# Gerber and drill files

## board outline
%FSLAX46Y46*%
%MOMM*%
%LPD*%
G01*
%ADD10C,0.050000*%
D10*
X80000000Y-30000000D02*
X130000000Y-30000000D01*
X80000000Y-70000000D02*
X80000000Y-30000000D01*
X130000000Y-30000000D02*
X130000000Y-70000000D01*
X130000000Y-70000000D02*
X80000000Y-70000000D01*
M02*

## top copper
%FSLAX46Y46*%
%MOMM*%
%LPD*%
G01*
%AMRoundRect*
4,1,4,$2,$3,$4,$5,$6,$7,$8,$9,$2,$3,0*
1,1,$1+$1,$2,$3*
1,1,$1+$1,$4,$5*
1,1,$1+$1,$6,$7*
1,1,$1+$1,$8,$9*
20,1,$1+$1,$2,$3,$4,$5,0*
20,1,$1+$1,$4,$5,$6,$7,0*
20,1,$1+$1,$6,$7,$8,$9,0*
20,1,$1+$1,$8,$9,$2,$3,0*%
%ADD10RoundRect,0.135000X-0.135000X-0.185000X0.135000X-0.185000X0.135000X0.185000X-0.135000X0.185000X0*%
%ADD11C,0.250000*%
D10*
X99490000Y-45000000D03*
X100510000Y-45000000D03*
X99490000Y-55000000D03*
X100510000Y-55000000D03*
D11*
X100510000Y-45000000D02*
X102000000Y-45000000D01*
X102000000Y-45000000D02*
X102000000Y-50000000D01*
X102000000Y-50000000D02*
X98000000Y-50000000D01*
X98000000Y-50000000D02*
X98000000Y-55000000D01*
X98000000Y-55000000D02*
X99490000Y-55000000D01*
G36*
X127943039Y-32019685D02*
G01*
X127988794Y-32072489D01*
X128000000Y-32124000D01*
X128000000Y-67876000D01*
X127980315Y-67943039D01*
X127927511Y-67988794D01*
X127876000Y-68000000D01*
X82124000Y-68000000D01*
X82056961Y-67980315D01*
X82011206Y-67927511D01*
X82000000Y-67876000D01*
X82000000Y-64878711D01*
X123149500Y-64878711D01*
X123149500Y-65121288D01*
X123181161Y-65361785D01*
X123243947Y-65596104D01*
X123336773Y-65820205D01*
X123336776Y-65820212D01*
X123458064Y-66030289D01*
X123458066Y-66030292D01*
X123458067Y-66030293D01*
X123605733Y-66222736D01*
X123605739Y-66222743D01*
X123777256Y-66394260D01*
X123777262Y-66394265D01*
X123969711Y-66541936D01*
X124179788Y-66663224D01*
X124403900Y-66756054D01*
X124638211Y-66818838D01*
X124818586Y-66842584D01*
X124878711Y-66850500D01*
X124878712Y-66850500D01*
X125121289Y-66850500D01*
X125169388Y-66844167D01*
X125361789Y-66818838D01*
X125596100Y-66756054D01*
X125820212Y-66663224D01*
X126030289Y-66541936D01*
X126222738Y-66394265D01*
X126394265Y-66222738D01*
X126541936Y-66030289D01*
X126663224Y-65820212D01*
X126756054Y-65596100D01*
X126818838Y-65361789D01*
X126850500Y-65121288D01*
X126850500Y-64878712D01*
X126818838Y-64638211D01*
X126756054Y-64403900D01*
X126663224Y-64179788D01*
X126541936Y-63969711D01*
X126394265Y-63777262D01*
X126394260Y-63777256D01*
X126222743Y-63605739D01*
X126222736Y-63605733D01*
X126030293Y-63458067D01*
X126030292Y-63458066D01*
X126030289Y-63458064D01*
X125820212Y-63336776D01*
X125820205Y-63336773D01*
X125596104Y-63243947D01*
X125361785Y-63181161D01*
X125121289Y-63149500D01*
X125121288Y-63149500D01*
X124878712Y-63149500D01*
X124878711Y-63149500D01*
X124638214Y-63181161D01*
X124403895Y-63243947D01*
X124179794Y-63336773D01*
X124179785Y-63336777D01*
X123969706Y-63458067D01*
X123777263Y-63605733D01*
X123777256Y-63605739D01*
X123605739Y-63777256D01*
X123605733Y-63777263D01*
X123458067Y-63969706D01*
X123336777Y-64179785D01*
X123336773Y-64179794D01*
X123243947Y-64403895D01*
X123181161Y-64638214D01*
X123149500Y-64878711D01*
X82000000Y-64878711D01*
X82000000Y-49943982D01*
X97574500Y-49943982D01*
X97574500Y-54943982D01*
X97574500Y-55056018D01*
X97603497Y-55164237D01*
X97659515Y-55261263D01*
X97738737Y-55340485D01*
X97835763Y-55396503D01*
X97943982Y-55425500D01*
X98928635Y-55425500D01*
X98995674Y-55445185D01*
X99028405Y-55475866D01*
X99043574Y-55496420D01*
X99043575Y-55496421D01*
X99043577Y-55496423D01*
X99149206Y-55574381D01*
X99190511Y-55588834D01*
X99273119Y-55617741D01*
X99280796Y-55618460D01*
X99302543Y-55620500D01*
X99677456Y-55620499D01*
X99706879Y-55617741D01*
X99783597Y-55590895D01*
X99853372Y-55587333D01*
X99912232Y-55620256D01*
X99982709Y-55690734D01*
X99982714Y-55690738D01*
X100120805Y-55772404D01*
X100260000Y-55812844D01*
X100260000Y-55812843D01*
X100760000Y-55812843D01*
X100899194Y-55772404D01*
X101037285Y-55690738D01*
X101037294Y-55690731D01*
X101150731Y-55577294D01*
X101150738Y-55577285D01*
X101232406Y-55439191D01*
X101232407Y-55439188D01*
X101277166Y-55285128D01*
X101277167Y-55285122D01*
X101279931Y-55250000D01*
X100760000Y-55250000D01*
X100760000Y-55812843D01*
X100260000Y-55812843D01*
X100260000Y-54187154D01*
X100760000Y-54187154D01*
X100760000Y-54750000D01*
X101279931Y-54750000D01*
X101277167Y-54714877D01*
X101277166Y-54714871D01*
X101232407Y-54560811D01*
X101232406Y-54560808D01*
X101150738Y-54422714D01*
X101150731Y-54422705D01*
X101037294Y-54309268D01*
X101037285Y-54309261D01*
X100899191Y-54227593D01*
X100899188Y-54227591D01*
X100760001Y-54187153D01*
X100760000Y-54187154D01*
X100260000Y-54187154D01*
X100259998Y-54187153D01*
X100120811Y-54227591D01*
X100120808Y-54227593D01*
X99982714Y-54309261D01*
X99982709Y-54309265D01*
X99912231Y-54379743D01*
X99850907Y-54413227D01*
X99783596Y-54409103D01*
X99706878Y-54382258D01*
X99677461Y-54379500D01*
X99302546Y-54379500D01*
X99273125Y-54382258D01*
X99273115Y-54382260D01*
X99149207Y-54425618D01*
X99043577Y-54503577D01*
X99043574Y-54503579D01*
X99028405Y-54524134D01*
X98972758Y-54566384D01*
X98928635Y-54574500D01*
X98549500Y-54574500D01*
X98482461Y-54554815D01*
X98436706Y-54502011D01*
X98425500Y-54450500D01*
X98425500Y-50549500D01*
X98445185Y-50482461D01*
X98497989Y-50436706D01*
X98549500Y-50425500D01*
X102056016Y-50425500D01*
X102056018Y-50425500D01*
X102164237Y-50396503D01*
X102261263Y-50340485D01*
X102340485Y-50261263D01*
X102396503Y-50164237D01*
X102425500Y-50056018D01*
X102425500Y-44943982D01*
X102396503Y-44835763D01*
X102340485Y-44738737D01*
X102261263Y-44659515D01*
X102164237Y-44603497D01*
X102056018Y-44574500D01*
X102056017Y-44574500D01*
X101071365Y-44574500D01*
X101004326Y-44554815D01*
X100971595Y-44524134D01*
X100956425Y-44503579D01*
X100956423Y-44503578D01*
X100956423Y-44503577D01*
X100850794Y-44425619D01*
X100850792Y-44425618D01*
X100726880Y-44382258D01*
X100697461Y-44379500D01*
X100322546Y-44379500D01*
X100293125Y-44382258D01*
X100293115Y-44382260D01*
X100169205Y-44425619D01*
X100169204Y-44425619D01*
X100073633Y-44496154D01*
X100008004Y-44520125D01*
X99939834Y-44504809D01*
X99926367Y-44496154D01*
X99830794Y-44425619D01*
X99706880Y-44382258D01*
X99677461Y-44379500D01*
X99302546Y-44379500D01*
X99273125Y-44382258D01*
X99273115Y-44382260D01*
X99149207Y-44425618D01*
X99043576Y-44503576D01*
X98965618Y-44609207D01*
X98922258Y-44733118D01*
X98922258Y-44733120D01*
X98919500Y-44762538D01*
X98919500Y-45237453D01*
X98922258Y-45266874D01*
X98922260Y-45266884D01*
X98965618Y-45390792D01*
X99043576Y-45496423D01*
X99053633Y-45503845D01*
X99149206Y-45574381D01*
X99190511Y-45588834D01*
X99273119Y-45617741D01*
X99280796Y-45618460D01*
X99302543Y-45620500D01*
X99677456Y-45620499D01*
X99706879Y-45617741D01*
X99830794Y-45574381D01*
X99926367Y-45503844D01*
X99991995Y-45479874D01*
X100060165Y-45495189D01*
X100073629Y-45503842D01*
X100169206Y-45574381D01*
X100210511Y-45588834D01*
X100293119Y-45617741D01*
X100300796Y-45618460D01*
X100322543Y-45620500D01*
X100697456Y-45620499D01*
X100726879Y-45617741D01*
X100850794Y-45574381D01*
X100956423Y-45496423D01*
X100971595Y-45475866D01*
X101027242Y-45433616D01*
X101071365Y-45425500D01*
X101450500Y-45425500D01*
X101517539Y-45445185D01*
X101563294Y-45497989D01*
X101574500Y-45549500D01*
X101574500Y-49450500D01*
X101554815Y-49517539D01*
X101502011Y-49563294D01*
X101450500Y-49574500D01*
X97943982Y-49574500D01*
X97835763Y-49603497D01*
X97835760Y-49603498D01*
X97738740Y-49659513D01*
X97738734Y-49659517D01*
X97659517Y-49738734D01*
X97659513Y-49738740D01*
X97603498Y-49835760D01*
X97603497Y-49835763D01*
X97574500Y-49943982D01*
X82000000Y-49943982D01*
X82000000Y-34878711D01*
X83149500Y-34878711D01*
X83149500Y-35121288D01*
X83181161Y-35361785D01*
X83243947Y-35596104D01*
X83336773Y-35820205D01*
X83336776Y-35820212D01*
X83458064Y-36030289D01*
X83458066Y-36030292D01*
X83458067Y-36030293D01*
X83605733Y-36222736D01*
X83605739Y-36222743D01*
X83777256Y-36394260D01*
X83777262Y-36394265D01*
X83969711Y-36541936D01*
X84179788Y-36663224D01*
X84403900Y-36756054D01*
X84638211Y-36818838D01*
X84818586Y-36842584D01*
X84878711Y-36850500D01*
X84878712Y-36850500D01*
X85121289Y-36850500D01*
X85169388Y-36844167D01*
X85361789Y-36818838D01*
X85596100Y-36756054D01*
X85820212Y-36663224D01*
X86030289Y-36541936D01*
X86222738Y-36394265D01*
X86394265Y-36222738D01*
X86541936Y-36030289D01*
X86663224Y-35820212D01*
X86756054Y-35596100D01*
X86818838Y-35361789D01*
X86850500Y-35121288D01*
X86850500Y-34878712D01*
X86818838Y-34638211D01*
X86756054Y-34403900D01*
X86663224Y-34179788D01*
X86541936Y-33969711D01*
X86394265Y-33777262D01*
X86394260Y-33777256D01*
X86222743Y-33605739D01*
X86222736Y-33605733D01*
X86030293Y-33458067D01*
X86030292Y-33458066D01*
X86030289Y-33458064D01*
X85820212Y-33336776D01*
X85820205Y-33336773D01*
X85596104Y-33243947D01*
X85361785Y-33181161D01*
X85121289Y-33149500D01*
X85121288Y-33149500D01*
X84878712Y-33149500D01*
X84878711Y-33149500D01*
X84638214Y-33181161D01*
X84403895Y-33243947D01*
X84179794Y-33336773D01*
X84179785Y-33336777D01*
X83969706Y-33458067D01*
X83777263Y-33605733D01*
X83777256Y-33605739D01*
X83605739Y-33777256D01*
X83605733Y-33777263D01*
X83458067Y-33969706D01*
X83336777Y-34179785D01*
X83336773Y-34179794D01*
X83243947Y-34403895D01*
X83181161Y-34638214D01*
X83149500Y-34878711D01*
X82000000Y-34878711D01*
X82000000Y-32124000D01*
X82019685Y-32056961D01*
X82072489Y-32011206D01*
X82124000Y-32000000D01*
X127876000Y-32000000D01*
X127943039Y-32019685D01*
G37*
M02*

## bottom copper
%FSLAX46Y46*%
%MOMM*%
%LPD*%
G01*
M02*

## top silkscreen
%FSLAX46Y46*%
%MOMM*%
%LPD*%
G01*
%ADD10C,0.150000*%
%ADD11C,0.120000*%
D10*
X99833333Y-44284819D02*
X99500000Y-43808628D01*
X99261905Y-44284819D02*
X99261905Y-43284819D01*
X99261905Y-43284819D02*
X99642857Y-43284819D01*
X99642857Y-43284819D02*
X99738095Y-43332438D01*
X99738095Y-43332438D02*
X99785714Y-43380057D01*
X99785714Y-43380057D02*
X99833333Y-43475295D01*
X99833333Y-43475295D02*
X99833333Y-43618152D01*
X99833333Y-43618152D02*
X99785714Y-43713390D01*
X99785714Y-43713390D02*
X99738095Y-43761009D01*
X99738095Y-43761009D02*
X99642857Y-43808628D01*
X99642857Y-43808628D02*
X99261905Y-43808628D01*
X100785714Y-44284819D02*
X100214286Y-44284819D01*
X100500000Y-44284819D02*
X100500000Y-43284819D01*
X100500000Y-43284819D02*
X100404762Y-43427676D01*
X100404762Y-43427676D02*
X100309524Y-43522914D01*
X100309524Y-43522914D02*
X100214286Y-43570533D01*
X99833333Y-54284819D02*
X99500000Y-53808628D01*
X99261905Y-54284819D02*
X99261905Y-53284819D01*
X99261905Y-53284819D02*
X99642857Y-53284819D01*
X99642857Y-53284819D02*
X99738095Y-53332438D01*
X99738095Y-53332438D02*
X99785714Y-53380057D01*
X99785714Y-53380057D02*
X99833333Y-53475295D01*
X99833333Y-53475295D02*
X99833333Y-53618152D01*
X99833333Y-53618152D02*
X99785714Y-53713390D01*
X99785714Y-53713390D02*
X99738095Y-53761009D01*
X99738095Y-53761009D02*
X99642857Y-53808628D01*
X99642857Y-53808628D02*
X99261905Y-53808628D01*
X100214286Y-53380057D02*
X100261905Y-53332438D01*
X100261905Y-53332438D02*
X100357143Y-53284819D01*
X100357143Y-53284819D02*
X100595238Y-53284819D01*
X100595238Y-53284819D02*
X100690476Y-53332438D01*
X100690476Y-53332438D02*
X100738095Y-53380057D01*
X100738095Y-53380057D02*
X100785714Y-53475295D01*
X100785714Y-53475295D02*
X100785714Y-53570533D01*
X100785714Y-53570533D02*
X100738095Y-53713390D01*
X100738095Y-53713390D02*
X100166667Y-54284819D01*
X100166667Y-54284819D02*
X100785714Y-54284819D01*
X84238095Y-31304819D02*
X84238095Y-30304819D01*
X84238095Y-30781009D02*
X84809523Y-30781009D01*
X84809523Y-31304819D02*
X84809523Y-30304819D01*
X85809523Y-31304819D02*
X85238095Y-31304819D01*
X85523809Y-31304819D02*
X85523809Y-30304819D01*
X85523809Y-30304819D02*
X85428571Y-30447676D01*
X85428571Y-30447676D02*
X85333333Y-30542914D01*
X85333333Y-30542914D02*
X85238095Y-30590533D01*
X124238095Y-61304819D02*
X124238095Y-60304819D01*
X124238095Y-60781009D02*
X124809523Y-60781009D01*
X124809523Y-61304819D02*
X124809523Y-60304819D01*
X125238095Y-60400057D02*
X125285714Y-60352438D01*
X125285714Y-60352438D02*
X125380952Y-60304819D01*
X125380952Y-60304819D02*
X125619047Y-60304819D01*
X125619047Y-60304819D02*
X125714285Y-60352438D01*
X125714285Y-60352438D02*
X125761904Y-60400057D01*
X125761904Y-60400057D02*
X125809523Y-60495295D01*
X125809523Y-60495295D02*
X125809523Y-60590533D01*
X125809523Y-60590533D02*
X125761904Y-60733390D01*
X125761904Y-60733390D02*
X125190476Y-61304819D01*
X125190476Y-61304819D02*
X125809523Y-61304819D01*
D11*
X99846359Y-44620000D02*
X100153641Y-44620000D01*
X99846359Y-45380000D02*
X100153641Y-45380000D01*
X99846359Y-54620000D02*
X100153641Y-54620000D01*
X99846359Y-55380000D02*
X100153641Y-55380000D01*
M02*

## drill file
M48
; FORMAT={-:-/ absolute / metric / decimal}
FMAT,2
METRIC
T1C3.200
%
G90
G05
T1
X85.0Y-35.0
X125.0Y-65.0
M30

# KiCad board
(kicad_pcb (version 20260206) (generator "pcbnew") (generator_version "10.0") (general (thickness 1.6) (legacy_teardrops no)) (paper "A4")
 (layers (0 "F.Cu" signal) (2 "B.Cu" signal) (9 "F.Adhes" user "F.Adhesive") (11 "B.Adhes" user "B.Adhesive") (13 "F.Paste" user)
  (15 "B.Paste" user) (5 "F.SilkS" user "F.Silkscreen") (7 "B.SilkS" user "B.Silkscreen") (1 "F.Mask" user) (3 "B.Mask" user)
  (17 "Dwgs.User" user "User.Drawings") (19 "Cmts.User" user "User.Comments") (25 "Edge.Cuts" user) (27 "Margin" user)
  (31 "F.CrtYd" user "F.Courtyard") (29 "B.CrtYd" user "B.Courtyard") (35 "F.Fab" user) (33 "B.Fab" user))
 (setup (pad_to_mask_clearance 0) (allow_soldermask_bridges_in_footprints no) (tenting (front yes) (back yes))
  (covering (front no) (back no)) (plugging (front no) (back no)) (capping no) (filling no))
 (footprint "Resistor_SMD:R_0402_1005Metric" (layer "F.Cu") (at 100 45)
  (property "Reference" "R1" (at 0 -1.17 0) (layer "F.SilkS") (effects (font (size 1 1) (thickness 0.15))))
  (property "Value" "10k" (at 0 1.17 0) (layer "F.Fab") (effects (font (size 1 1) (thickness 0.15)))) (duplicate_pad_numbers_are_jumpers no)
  (fp_line (start -0.153641 -0.38) (end 0.153641 -0.38) (stroke (width 0.12) (type solid)) (layer "F.SilkS"))
  (fp_line (start -0.153641 0.38) (end 0.153641 0.38) (stroke (width 0.12) (type solid)) (layer "F.SilkS"))
  (pad "1" smd roundrect (at -0.51 0) (size 0.54 0.64) (layers "F.Cu" "F.Mask" "F.Paste") (roundrect_rratio 0.25) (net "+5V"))
  (pad "2" smd roundrect (at 0.51 0) (size 0.54 0.64) (layers "F.Cu" "F.Mask" "F.Paste") (roundrect_rratio 0.25) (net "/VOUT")))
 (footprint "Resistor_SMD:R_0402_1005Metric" (layer "F.Cu") (at 100 55)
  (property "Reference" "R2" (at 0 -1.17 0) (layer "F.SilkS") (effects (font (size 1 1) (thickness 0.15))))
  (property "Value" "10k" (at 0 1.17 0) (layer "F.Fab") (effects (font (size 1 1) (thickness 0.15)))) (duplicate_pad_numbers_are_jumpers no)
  (fp_line (start -0.153641 -0.38) (end 0.153641 -0.38) (stroke (width 0.12) (type solid)) (layer "F.SilkS"))
  (fp_line (start -0.153641 0.38) (end 0.153641 0.38) (stroke (width 0.12) (type solid)) (layer "F.SilkS"))
  (pad "1" smd roundrect (at -0.51 0) (size 0.54 0.64) (layers "F.Cu" "F.Mask" "F.Paste") (roundrect_rratio 0.25) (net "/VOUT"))
  (pad "2" smd roundrect (at 0.51 0) (size 0.54 0.64) (layers "F.Cu" "F.Mask" "F.Paste") (roundrect_rratio 0.25) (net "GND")))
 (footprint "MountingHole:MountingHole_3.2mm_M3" (layer "F.Cu") (at 85 35)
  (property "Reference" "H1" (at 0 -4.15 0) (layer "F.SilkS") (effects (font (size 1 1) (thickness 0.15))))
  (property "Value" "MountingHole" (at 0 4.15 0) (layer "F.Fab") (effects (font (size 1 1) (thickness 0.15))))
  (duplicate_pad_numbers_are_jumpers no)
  (pad "" np_thru_hole circle (at 0 0) (size 3.2 3.2) (drill 3.2) (layers "*.Cu" "*.Mask")))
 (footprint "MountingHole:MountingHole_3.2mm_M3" (layer "F.Cu") (at 125 65)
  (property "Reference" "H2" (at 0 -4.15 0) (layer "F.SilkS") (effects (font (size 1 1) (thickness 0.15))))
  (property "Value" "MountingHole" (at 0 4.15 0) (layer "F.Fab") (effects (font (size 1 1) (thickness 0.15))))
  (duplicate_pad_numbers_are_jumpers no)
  (pad "" np_thru_hole circle (at 0 0) (size 3.2 3.2) (drill 3.2) (layers "*.Cu" "*.Mask")))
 (gr_line (start 80 30) (end 130 30) (stroke (width 0.05) (type default)) (layer "Edge.Cuts"))
 (gr_line (start 80 70) (end 80 30) (stroke (width 0.05) (type default)) (layer "Edge.Cuts"))
 (gr_line (start 130 30) (end 130 70) (stroke (width 0.05) (type default)) (layer "Edge.Cuts"))
 (gr_line (start 130 70) (end 80 70) (stroke (width 0.05) (type default)) (layer "Edge.Cuts"))
 (segment (start 100.51 45) (end 102 45) (width 0.25) (layer "F.Cu") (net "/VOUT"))
 (segment (start 102 45) (end 102 50) (width 0.25) (layer "F.Cu") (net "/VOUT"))
 (segment (start 102 50) (end 98 50) (width 0.25) (layer "F.Cu") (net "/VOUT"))
 (segment (start 98 50) (end 98 55) (width 0.25) (layer "F.Cu") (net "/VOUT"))
 (segment (start 98 55) (end 99.49 55) (width 0.25) (layer "F.Cu") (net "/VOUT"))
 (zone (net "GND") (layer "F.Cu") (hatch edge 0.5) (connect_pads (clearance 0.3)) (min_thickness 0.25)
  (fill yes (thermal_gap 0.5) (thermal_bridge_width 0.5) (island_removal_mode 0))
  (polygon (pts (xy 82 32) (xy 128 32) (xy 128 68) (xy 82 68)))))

